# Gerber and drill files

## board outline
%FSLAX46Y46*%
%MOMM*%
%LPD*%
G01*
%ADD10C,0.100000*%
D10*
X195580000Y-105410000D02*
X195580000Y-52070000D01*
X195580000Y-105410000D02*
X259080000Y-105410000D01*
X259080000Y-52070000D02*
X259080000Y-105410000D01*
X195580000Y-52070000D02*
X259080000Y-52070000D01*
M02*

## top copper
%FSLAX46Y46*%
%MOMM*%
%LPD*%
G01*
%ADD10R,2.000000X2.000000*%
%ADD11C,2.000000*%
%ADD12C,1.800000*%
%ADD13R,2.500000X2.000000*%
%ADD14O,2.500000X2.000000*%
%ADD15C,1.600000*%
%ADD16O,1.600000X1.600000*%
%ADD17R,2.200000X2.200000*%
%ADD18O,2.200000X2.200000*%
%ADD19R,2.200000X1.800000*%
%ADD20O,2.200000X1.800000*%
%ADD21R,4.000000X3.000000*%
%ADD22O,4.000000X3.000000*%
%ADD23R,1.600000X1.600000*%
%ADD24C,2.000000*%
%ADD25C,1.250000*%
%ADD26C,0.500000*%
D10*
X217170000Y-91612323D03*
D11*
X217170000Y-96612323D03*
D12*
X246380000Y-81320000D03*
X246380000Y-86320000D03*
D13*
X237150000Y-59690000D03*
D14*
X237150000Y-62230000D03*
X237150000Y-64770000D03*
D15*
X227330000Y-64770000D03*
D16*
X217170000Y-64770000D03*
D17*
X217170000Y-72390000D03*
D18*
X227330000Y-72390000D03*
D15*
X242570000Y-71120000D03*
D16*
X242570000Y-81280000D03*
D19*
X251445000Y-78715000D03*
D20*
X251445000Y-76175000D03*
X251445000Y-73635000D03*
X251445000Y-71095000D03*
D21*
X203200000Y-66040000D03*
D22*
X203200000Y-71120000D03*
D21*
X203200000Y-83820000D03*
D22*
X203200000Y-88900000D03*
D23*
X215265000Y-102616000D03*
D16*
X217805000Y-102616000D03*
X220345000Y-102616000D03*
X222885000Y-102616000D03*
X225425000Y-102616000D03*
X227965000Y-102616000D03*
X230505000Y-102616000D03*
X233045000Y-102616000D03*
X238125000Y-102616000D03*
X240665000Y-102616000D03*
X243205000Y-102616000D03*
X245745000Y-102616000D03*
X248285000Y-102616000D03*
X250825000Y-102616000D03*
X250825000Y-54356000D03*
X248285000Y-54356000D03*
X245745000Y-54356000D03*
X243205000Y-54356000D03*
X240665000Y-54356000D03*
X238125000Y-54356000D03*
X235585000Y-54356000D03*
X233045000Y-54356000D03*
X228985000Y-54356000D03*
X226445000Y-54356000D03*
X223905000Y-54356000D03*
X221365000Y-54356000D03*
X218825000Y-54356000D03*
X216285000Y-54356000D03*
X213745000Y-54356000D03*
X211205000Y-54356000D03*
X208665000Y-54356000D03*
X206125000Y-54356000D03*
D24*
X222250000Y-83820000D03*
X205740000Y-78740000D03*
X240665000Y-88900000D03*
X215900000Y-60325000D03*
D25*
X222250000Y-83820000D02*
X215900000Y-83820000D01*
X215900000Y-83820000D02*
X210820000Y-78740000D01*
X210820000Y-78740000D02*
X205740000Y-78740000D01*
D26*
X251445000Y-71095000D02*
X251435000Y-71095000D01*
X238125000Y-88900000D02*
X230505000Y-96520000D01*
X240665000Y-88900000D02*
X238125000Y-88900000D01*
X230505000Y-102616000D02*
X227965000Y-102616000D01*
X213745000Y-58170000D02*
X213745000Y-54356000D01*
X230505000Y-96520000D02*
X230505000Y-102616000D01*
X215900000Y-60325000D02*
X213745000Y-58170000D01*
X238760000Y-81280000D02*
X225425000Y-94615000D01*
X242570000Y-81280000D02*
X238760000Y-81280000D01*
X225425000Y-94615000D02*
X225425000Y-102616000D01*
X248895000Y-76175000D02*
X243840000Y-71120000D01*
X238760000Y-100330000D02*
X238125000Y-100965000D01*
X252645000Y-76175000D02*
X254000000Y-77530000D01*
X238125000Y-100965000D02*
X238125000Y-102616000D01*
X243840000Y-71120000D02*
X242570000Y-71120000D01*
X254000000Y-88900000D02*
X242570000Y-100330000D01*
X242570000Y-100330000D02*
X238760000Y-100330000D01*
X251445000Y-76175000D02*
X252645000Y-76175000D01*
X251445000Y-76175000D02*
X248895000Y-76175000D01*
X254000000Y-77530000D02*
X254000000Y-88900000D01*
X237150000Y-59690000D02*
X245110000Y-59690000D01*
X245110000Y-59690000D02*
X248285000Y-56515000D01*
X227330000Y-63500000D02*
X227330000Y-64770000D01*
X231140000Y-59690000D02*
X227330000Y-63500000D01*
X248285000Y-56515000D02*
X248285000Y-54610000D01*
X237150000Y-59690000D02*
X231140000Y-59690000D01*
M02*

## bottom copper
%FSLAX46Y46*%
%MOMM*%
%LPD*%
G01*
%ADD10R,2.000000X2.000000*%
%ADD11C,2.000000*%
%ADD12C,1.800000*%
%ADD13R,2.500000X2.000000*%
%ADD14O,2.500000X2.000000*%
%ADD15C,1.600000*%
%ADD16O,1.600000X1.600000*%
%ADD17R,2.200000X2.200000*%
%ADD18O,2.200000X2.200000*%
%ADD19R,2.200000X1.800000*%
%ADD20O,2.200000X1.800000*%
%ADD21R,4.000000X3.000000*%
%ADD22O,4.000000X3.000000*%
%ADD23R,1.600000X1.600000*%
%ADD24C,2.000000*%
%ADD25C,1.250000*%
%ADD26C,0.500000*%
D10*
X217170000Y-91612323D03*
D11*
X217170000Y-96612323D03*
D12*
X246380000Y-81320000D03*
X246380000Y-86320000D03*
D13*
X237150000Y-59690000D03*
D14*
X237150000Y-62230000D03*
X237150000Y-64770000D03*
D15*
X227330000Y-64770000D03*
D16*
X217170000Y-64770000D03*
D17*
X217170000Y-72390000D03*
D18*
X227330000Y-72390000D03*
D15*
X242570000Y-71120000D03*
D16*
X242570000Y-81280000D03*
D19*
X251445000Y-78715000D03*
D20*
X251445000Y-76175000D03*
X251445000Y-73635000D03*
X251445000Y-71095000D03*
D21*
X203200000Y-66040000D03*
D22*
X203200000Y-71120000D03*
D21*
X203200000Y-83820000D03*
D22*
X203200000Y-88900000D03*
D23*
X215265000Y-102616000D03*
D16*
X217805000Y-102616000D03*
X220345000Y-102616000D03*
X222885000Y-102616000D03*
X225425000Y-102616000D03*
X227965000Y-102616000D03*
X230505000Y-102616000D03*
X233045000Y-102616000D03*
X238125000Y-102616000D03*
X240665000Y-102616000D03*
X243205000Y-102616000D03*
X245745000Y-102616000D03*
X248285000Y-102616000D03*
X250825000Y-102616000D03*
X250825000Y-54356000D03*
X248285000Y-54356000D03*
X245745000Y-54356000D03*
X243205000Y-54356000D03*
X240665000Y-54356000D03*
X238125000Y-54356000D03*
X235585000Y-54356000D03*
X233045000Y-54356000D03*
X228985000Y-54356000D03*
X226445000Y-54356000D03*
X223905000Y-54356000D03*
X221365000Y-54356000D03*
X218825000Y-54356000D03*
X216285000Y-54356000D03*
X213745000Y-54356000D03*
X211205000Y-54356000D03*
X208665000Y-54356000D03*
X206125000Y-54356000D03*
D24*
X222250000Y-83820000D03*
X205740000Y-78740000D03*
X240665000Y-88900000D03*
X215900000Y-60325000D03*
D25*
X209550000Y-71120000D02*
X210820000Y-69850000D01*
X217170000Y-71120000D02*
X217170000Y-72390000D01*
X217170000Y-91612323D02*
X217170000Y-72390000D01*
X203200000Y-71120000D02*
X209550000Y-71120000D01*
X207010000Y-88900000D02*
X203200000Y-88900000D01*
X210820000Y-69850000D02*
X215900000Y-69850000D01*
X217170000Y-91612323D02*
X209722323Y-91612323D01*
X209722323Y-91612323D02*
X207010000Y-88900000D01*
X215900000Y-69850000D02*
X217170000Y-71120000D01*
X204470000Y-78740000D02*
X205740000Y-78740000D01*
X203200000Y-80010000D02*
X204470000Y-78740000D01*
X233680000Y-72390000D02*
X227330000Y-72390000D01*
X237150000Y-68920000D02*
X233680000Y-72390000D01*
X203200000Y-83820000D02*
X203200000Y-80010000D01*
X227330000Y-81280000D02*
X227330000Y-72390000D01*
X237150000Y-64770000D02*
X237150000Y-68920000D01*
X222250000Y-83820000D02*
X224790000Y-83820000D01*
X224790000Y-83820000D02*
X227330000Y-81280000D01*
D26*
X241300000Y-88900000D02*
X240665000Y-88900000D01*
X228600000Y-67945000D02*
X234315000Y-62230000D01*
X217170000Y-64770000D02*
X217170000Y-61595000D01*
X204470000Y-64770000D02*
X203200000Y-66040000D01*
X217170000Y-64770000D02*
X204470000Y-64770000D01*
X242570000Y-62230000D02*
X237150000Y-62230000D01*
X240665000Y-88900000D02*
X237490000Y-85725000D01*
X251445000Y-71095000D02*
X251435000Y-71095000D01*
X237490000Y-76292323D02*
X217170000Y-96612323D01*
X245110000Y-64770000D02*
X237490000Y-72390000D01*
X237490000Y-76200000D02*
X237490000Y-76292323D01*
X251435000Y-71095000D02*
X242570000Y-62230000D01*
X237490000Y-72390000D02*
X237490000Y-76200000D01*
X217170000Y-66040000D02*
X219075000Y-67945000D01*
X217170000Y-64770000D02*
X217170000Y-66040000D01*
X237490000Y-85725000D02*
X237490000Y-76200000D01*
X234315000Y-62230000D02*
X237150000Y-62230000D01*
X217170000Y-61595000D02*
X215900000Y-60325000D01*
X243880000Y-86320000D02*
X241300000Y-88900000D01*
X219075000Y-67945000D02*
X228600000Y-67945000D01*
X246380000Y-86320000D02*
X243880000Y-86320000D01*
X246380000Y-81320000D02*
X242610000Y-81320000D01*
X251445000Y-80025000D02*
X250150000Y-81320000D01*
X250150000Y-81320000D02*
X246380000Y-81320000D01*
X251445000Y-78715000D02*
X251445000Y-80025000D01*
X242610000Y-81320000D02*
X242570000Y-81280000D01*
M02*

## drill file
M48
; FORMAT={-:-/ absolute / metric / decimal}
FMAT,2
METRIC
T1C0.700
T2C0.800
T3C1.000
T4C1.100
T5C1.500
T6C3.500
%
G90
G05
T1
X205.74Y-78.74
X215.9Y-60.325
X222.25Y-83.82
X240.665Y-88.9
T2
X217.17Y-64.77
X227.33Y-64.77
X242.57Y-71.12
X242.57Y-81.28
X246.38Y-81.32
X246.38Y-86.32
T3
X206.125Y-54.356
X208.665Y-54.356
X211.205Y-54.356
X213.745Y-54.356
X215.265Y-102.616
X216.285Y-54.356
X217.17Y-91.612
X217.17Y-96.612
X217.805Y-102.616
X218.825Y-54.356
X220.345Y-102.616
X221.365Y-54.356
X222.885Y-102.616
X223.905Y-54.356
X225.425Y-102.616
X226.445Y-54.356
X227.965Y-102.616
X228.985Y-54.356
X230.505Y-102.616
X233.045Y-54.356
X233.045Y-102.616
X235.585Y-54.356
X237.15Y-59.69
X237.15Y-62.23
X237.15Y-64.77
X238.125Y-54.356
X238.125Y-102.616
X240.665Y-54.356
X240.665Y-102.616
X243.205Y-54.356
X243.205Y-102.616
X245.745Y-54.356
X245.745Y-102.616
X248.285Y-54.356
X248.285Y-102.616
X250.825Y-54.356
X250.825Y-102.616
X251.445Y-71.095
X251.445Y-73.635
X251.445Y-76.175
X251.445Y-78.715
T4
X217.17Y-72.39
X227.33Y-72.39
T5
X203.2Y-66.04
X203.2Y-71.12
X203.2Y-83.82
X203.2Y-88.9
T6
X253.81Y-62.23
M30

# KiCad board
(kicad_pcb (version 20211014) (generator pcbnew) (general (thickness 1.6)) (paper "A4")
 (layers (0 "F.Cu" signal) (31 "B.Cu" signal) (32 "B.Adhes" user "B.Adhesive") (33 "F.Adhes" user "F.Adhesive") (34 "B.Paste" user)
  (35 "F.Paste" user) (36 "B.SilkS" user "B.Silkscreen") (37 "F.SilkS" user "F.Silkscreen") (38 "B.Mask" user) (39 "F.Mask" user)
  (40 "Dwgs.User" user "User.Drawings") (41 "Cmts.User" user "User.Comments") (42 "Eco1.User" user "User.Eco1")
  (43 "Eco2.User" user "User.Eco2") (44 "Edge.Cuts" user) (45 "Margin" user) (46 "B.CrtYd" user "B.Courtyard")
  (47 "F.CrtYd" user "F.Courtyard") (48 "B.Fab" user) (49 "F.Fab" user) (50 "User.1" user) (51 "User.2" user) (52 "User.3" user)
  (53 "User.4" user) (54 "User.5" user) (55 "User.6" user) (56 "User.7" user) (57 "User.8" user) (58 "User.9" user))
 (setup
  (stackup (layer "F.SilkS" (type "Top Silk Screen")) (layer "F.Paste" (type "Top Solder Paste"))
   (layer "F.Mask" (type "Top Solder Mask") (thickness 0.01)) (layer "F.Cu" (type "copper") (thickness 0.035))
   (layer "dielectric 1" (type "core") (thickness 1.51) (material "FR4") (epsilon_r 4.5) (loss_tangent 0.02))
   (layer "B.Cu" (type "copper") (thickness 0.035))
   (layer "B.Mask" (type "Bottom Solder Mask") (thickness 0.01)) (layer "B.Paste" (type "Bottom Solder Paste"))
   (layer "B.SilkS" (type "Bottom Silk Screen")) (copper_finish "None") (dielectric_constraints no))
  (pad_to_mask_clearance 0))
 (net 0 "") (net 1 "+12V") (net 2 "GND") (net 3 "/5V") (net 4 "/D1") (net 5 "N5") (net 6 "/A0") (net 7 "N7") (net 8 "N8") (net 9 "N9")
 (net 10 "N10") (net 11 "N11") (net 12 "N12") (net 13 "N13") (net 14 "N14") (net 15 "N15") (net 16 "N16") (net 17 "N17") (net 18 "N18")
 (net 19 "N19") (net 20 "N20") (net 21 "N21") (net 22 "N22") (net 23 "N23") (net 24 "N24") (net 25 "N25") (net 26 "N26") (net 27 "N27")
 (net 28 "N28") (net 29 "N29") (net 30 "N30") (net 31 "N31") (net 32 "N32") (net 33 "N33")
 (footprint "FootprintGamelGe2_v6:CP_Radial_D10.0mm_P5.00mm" (layer "F.Cu") (at 217.17 91.612323 -90)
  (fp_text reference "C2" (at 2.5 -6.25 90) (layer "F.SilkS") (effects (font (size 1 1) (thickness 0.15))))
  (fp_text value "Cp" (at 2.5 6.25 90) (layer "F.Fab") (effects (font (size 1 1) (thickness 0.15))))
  (pad "1" thru_hole rect (at 0 0 270) (size 2 2) (drill 1) (layers *.Cu *.Mask) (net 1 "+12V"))
  (pad "2" thru_hole circle (at 5 0 270) (size 2 2) (drill 1) (layers *.Cu *.Mask) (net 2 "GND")))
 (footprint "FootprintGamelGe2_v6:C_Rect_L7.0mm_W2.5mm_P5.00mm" (layer "F.Cu") (at 246.38 81.32 -90)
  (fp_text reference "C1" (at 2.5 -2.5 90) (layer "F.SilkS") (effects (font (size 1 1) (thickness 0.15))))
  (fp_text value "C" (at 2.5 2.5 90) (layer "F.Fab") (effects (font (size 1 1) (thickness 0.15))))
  (pad "1" thru_hole circle (at 0 0 270) (size 1.8 1.8) (drill 0.8) (layers *.Cu *.Mask) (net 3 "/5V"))
  (pad "2" thru_hole circle (at 5 0 270) (size 1.8 1.8) (drill 0.8) (layers *.Cu *.Mask) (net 2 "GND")))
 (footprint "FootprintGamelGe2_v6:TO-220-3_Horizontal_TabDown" (layer "F.Cu") (at 237.15 59.69 -90)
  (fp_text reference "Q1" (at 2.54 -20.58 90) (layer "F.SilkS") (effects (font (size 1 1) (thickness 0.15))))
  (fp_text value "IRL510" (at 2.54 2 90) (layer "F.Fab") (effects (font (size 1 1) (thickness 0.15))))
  (pad "" np_thru_hole oval (at 2.54 -16.66 270) (size 3.5 3.5) (drill 3.5) (layers *.Cu *.Mask))
  (pad "1" thru_hole rect (at 0 0 270) (size 2 2.5) (drill 1) (layers *.Cu *.Mask) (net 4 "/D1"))
  (pad "2" thru_hole oval (at 2.54 0 270) (size 2 2.5) (drill 1) (layers *.Cu *.Mask) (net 2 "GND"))
  (pad "3" thru_hole oval (at 5.08 0 270) (size 2 2.5) (drill 1) (layers *.Cu *.Mask) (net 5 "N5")))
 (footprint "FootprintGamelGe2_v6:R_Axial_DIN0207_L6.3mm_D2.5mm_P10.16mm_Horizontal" (layer "F.Cu") (at 227.33 64.77 180)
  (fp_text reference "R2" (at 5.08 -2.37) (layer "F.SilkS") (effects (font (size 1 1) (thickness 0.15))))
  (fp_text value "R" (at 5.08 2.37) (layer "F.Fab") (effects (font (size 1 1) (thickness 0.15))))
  (pad "1" thru_hole circle (at 0 0 180) (size 1.6 1.6) (drill 0.8) (layers *.Cu *.Mask) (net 4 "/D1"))
  (pad "2" thru_hole oval (at 10.16 0 180) (size 1.6 1.6) (drill 0.8) (layers *.Cu *.Mask) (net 2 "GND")))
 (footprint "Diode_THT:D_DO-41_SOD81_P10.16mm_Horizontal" (layer "F.Cu") (at 217.17 72.39)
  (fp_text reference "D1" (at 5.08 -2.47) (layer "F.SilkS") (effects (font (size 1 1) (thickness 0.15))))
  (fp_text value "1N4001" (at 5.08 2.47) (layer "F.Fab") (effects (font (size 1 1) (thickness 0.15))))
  (pad "1" thru_hole rect (at 0 0) (size 2.2 2.2) (drill 1.1) (layers *.Cu *.Mask) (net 1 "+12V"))
  (pad "2" thru_hole oval (at 10.16 0) (size 2.2 2.2) (drill 1.1) (layers *.Cu *.Mask) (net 5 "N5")))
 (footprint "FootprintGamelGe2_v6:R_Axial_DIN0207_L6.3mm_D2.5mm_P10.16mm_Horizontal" (layer "F.Cu") (at 242.57 71.12 -90)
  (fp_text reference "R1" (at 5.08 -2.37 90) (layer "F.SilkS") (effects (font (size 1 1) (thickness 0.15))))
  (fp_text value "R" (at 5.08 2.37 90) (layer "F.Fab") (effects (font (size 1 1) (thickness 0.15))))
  (pad "1" thru_hole circle (at 0 0 270) (size 1.6 1.6) (drill 0.8) (layers *.Cu *.Mask) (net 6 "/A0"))
  (pad "2" thru_hole oval (at 10.16 0 270) (size 1.6 1.6) (drill 0.8) (layers *.Cu *.Mask) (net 3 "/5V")))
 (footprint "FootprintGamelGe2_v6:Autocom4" (layer "F.Cu") (at 251.445 78.715 180)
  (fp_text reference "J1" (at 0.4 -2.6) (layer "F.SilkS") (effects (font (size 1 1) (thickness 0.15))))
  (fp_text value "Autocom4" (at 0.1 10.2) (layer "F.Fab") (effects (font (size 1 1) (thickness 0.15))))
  (pad "1" thru_hole rect (at 0 0 180) (size 2.2 1.8) (drill 1) (layers *.Cu *.Mask) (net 3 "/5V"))
  (pad "2" thru_hole oval (at 0 2.54 180) (size 2.2 1.8) (drill 1) (layers *.Cu *.Mask) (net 6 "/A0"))
  (pad "3" thru_hole oval (at 0 5.08 180) (size 2.2 1.8) (drill 1) (layers *.Cu *.Mask) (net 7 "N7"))
  (pad "4" thru_hole oval (at 0 7.62 180) (size 2.2 1.8) (drill 1) (layers *.Cu *.Mask) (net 2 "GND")))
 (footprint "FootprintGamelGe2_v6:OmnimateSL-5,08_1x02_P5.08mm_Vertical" (layer "F.Cu") (at 203.2 66.04 -90)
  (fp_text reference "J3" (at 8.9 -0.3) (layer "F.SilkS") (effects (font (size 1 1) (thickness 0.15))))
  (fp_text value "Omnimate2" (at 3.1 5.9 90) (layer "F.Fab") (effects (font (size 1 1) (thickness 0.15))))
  (pad "1" thru_hole rect (at 0 0 270) (size 3 4) (drill 1.5) (layers *.Cu *.Mask) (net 2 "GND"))
  (pad "2" thru_hole oval (at 5.08 0 270) (size 3 4) (drill 1.5) (layers *.Cu *.Mask) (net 1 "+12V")))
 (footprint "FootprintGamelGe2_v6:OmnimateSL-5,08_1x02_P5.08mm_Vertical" (layer "F.Cu") (at 203.2 83.82 -90)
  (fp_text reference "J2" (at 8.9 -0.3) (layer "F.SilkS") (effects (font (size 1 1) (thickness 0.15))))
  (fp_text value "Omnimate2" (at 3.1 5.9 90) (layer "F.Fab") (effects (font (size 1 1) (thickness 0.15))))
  (pad "1" thru_hole rect (at 0 0 270) (size 3 4) (drill 1.5) (layers *.Cu *.Mask) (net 5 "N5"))
  (pad "2" thru_hole oval (at 5.08 0 270) (size 3 4) (drill 1.5) (layers *.Cu *.Mask) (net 1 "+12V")))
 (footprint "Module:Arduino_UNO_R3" (layer "B.Cu") (at 215.265 102.616)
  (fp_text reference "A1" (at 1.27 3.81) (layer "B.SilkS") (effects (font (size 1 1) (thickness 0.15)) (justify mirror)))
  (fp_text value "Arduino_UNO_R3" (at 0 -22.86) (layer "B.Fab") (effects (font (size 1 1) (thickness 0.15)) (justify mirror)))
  (pad "1" thru_hole rect (at 0 0 270) (size 1.6 1.6) (drill 1) (layers *.Cu *.Mask) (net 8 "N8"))
  (pad "2" thru_hole oval (at 2.54 0 270) (size 1.6 1.6) (drill 1) (layers *.Cu *.Mask) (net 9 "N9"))
  (pad "3" thru_hole oval (at 5.08 0 270) (size 1.6 1.6) (drill 1) (layers *.Cu *.Mask) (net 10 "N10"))
  (pad "4" thru_hole oval (at 7.62 0 270) (size 1.6 1.6) (drill 1) (layers *.Cu *.Mask) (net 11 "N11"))
  (pad "5" thru_hole oval (at 10.16 0 270) (size 1.6 1.6) (drill 1) (layers *.Cu *.Mask) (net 3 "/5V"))
  (pad "6" thru_hole oval (at 12.7 0 270) (size 1.6 1.6) (drill 1) (layers *.Cu *.Mask) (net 2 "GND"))
  (pad "7" thru_hole oval (at 15.24 0 270) (size 1.6 1.6) (drill 1) (layers *.Cu *.Mask) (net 2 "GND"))
  (pad "8" thru_hole oval (at 17.78 0 270) (size 1.6 1.6) (drill 1) (layers *.Cu *.Mask) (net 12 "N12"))
  (pad "9" thru_hole oval (at 22.86 0 270) (size 1.6 1.6) (drill 1) (layers *.Cu *.Mask) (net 6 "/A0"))
  (pad "10" thru_hole oval (at 25.4 0 270) (size 1.6 1.6) (drill 1) (layers *.Cu *.Mask) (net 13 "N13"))
  (pad "11" thru_hole oval (at 27.94 0 270) (size 1.6 1.6) (drill 1) (layers *.Cu *.Mask) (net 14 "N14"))
  (pad "12" thru_hole oval (at 30.48 0 270) (size 1.6 1.6) (drill 1) (layers *.Cu *.Mask) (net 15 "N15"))
  (pad "13" thru_hole oval (at 33.02 0 270) (size 1.6 1.6) (drill 1) (layers *.Cu *.Mask) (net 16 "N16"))
  (pad "14" thru_hole oval (at 35.56 0 270) (size 1.6 1.6) (drill 1) (layers *.Cu *.Mask) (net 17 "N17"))
  (pad "15" thru_hole oval (at 35.56 -48.26 270) (size 1.6 1.6) (drill 1) (layers *.Cu *.Mask) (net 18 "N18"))
  (pad "16" thru_hole oval (at 33.02 -48.26 270) (size 1.6 1.6) (drill 1) (layers *.Cu *.Mask) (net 4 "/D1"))
  (pad "17" thru_hole oval (at 30.48 -48.26 270) (size 1.6 1.6) (drill 1) (layers *.Cu *.Mask) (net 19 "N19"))
  (pad "18" thru_hole oval (at 27.94 -48.26 270) (size 1.6 1.6) (drill 1) (layers *.Cu *.Mask) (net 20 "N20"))
  (pad "19" thru_hole oval (at 25.4 -48.26 270) (size 1.6 1.6) (drill 1) (layers *.Cu *.Mask) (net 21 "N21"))
  (pad "20" thru_hole oval (at 22.86 -48.26 270) (size 1.6 1.6) (drill 1) (layers *.Cu *.Mask) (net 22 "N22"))
  (pad "21" thru_hole oval (at 20.32 -48.26 270) (size 1.6 1.6) (drill 1) (layers *.Cu *.Mask) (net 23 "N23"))
  (pad "22" thru_hole oval (at 17.78 -48.26 270) (size 1.6 1.6) (drill 1) (layers *.Cu *.Mask) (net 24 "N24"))
  (pad "23" thru_hole oval (at 13.72 -48.26 270) (size 1.6 1.6) (drill 1) (layers *.Cu *.Mask) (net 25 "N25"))
  (pad "24" thru_hole oval (at 11.18 -48.26 270) (size 1.6 1.6) (drill 1) (layers *.Cu *.Mask) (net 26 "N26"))
  (pad "25" thru_hole oval (at 8.64 -48.26 270) (size 1.6 1.6) (drill 1) (layers *.Cu *.Mask) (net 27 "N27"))
  (pad "26" thru_hole oval (at 6.1 -48.26 270) (size 1.6 1.6) (drill 1) (layers *.Cu *.Mask) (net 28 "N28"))
  (pad "27" thru_hole oval (at 3.56 -48.26 270) (size 1.6 1.6) (drill 1) (layers *.Cu *.Mask) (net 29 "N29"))
  (pad "28" thru_hole oval (at 1.02 -48.26 270) (size 1.6 1.6) (drill 1) (layers *.Cu *.Mask) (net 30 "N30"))
  (pad "29" thru_hole oval (at -1.52 -48.26 270) (size 1.6 1.6) (drill 1) (layers *.Cu *.Mask) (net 2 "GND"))
  (pad "30" thru_hole oval (at -4.06 -48.26 270) (size 1.6 1.6) (drill 1) (layers *.Cu *.Mask) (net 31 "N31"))
  (pad "31" thru_hole oval (at -6.6 -48.26 270) (size 1.6 1.6) (drill 1) (layers *.Cu *.Mask) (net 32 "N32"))
  (pad "32" thru_hole oval (at -9.14 -48.26 270) (size 1.6 1.6) (drill 1) (layers *.Cu *.Mask) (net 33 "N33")))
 (gr_line (start 195.58 105.41) (end 195.58 52.07) (layer "Edge.Cuts") (width 0.1))
 (gr_line (start 195.58 105.41) (end 259.08 105.41) (layer "Edge.Cuts") (width 0.1))
 (gr_line (start 259.08 52.07) (end 259.08 105.41) (layer "Edge.Cuts") (width 0.1))
 (gr_line (start 195.58 52.07) (end 259.08 52.07) (layer "Edge.Cuts") (width 0.1))
 (segment (start 209.55 71.12) (end 210.82 69.85) (width 1.25) (layer "B.Cu") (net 1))
 (segment (start 217.17 71.12) (end 217.17 72.39) (width 1.25) (layer "B.Cu") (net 1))
 (segment (start 217.17 91.612323) (end 217.17 72.39) (width 1.25) (layer "B.Cu") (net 1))
 (segment (start 203.2 71.12) (end 209.55 71.12) (width 1.25) (layer "B.Cu") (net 1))
 (segment (start 207.01 88.9) (end 203.2 88.9) (width 1.25) (layer "B.Cu") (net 1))
 (segment (start 210.82 69.85) (end 215.9 69.85) (width 1.25) (layer "B.Cu") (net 1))
 (segment (start 217.17 91.612323) (end 209.722323 91.612323) (width 1.25) (layer "B.Cu") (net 1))
 (segment (start 209.722323 91.612323) (end 207.01 88.9) (width 1.25) (layer "B.Cu") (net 1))
 (segment (start 215.9 69.85) (end 217.17 71.12) (width 1.25) (layer "B.Cu") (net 1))
 (segment (start 222.25 83.82) (end 215.9 83.82) (width 1.25) (layer "F.Cu") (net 5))
 (segment (start 215.9 83.82) (end 210.82 78.74) (width 1.25) (layer "F.Cu") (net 5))
 (segment (start 210.82 78.74) (end 205.74 78.74) (width 1.25) (layer "F.Cu") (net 5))
 (via (at 222.25 83.82) (size 2) (drill 0.7) (layers "F.Cu" "B.Cu") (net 5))
 (via (at 205.74 78.74) (size 2) (drill 0.7) (layers "F.Cu" "B.Cu") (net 5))
 (segment (start 204.47 78.74) (end 205.74 78.74) (width 1.25) (layer "B.Cu") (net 5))
 (segment (start 203.2 80.01) (end 204.47 78.74) (width 1.25) (layer "B.Cu") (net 5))
 (segment (start 233.68 72.39) (end 227.33 72.39) (width 1.25) (layer "B.Cu") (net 5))
 (segment (start 237.15 68.92) (end 233.68 72.39) (width 1.25) (layer "B.Cu") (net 5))
 (segment (start 203.2 83.82) (end 203.2 80.01) (width 1.25) (layer "B.Cu") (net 5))
 (segment (start 227.33 81.28) (end 227.33 72.39) (width 1.25) (layer "B.Cu") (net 5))
 (segment (start 237.15 64.77) (end 237.15 68.92) (width 1.25) (layer "B.Cu") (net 5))
 (segment (start 222.25 83.82) (end 224.79 83.82) (width 1.25) (layer "B.Cu") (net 5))
 (segment (start 224.79 83.82) (end 227.33 81.28) (width 1.25) (layer "B.Cu") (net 5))
 (segment (start 251.445 71.095) (end 251.435 71.095) (width 0.5) (layer "F.Cu") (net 2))
 (segment (start 238.125 88.9) (end 230.505 96.52) (width 0.5) (layer "F.Cu") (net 2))
 (segment (start 240.665 88.9) (end 238.125 88.9) (width 0.5) (layer "F.Cu") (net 2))
 (segment (start 230.505 102.616) (end 227.965 102.616) (width 0.5) (layer "F.Cu") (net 2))
 (segment (start 213.745 58.17) (end 213.745 54.356) (width 0.5) (layer "F.Cu") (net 2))
 (segment (start 230.505 96.52) (end 230.505 102.616) (width 0.5) (layer "F.Cu") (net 2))
 (segment (start 215.9 60.325) (end 213.745 58.17) (width 0.5) (layer "F.Cu") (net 2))
 (via (at 240.665 88.9) (size 2) (drill 0.7) (layers "F.Cu" "B.Cu") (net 2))
 (via (at 215.9 60.325) (size 2) (drill 0.7) (layers "F.Cu" "B.Cu") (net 2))
 (segment (start 241.3 88.9) (end 240.665 88.9) (width 0.5) (layer "B.Cu") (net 2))
 (segment (start 228.6 67.945) (end 234.315 62.23) (width 0.5) (layer "B.Cu") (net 2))
 (segment (start 217.17 64.77) (end 217.17 61.595) (width 0.5) (layer "B.Cu") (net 2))
 (segment (start 204.47 64.77) (end 203.2 66.04) (width 0.5) (layer "B.Cu") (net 2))
 (segment (start 217.17 64.77) (end 204.47 64.77) (width 0.5) (layer "B.Cu") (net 2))
 (segment (start 242.57 62.23) (end 237.15 62.23) (width 0.5) (layer "B.Cu") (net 2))
 (segment (start 240.665 88.9) (end 237.49 85.725) (width 0.5) (layer "B.Cu") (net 2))
 (segment (start 251.445 71.095) (end 251.435 71.095) (width 0.5) (layer "B.Cu") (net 2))
 (segment (start 237.49 76.292323) (end 217.17 96.612323) (width 0.5) (layer "B.Cu") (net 2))
 (segment (start 245.11 64.77) (end 237.49 72.39) (width 0.5) (layer "B.Cu") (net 2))
 (segment (start 237.49 76.2) (end 237.49 76.292323) (width 0.5) (layer "B.Cu") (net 2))
 (segment (start 251.435 71.095) (end 242.57 62.23) (width 0.5) (layer "B.Cu") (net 2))
 (segment (start 237.49 72.39) (end 237.49 76.2) (width 0.5) (layer "B.Cu") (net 2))
 (segment (start 217.17 66.04) (end 219.075 67.945) (width 0.5) (layer "B.Cu") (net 2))
 (segment (start 217.17 64.77) (end 217.17 66.04) (width 0.5) (layer "B.Cu") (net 2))
 (segment (start 237.49 85.725) (end 237.49 76.2) (width 0.5) (layer "B.Cu") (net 2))
 (segment (start 234.315 62.23) (end 237.15 62.23) (width 0.5) (layer "B.Cu") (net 2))
 (segment (start 217.17 61.595) (end 215.9 60.325) (width 0.5) (layer "B.Cu") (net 2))
 (segment (start 243.88 86.32) (end 241.3 88.9) (width 0.5) (layer "B.Cu") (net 2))
 (segment (start 219.075 67.945) (end 228.6 67.945) (width 0.5) (layer "B.Cu") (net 2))
 (segment (start 246.38 86.32) (end 243.88 86.32) (width 0.5) (layer "B.Cu") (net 2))
 (segment (start 238.76 81.28) (end 225.425 94.615) (width 0.5) (layer "F.Cu") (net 3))
 (segment (start 242.57 81.28) (end 238.76 81.28) (width 0.5) (layer "F.Cu") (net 3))
 (segment (start 225.425 94.615) (end 225.425 102.616) (width 0.5) (layer "F.Cu") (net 3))
 (segment (start 246.38 81.32) (end 242.61 81.32) (width 0.5) (layer "B.Cu") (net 3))
 (segment (start 251.445 80.025) (end 250.15 81.32) (width 0.5) (layer "B.Cu") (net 3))
 (segment (start 250.15 81.32) (end 246.38 81.32) (width 0.5) (layer "B.Cu") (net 3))
 (segment (start 251.445 78.715) (end 251.445 80.025) (width 0.5) (layer "B.Cu") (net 3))
 (segment (start 242.61 81.32) (end 242.57 81.28) (width 0.5) (layer "B.Cu") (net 3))
 (segment (start 248.895 76.175) (end 243.84 71.12) (width 0.5) (layer "F.Cu") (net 6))
 (segment (start 238.76 100.33) (end 238.125 100.965) (width 0.5) (layer "F.Cu") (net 6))
 (segment (start 252.645 76.175) (end 254 77.53) (width 0.5) (layer "F.Cu") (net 6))
 (segment (start 238.125 100.965) (end 238.125 102.616) (width 0.5) (layer "F.Cu") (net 6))
 (segment (start 243.84 71.12) (end 242.57 71.12) (width 0.5) (layer "F.Cu") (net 6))
 (segment (start 254 88.9) (end 242.57 100.33) (width 0.5) (layer "F.Cu") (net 6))
 (segment (start 242.57 100.33) (end 238.76 100.33) (width 0.5) (layer "F.Cu") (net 6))
 (segment (start 251.445 76.175) (end 252.645 76.175) (width 0.5) (layer "F.Cu") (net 6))
 (segment (start 251.445 76.175) (end 248.895 76.175) (width 0.5) (layer "F.Cu") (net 6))
 (segment (start 254 77.53) (end 254 88.9) (width 0.5) (layer "F.Cu") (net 6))
 (segment (start 237.15 59.69) (end 245.11 59.69) (width 0.5) (layer "F.Cu") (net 4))
 (segment (start 245.11 59.69) (end 248.285 56.515) (width 0.5) (layer "F.Cu") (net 4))
 (segment (start 227.33 63.5) (end 227.33 64.77) (width 0.5) (layer "F.Cu") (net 4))
 (segment (start 231.14 59.69) (end 227.33 63.5) (width 0.5) (layer "F.Cu") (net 4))
 (segment (start 248.285 56.515) (end 248.285 54.61) (width 0.5) (layer "F.Cu") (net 4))
 (segment (start 237.15 59.69) (end 231.14 59.69) (width 0.5) (layer "F.Cu") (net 4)))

